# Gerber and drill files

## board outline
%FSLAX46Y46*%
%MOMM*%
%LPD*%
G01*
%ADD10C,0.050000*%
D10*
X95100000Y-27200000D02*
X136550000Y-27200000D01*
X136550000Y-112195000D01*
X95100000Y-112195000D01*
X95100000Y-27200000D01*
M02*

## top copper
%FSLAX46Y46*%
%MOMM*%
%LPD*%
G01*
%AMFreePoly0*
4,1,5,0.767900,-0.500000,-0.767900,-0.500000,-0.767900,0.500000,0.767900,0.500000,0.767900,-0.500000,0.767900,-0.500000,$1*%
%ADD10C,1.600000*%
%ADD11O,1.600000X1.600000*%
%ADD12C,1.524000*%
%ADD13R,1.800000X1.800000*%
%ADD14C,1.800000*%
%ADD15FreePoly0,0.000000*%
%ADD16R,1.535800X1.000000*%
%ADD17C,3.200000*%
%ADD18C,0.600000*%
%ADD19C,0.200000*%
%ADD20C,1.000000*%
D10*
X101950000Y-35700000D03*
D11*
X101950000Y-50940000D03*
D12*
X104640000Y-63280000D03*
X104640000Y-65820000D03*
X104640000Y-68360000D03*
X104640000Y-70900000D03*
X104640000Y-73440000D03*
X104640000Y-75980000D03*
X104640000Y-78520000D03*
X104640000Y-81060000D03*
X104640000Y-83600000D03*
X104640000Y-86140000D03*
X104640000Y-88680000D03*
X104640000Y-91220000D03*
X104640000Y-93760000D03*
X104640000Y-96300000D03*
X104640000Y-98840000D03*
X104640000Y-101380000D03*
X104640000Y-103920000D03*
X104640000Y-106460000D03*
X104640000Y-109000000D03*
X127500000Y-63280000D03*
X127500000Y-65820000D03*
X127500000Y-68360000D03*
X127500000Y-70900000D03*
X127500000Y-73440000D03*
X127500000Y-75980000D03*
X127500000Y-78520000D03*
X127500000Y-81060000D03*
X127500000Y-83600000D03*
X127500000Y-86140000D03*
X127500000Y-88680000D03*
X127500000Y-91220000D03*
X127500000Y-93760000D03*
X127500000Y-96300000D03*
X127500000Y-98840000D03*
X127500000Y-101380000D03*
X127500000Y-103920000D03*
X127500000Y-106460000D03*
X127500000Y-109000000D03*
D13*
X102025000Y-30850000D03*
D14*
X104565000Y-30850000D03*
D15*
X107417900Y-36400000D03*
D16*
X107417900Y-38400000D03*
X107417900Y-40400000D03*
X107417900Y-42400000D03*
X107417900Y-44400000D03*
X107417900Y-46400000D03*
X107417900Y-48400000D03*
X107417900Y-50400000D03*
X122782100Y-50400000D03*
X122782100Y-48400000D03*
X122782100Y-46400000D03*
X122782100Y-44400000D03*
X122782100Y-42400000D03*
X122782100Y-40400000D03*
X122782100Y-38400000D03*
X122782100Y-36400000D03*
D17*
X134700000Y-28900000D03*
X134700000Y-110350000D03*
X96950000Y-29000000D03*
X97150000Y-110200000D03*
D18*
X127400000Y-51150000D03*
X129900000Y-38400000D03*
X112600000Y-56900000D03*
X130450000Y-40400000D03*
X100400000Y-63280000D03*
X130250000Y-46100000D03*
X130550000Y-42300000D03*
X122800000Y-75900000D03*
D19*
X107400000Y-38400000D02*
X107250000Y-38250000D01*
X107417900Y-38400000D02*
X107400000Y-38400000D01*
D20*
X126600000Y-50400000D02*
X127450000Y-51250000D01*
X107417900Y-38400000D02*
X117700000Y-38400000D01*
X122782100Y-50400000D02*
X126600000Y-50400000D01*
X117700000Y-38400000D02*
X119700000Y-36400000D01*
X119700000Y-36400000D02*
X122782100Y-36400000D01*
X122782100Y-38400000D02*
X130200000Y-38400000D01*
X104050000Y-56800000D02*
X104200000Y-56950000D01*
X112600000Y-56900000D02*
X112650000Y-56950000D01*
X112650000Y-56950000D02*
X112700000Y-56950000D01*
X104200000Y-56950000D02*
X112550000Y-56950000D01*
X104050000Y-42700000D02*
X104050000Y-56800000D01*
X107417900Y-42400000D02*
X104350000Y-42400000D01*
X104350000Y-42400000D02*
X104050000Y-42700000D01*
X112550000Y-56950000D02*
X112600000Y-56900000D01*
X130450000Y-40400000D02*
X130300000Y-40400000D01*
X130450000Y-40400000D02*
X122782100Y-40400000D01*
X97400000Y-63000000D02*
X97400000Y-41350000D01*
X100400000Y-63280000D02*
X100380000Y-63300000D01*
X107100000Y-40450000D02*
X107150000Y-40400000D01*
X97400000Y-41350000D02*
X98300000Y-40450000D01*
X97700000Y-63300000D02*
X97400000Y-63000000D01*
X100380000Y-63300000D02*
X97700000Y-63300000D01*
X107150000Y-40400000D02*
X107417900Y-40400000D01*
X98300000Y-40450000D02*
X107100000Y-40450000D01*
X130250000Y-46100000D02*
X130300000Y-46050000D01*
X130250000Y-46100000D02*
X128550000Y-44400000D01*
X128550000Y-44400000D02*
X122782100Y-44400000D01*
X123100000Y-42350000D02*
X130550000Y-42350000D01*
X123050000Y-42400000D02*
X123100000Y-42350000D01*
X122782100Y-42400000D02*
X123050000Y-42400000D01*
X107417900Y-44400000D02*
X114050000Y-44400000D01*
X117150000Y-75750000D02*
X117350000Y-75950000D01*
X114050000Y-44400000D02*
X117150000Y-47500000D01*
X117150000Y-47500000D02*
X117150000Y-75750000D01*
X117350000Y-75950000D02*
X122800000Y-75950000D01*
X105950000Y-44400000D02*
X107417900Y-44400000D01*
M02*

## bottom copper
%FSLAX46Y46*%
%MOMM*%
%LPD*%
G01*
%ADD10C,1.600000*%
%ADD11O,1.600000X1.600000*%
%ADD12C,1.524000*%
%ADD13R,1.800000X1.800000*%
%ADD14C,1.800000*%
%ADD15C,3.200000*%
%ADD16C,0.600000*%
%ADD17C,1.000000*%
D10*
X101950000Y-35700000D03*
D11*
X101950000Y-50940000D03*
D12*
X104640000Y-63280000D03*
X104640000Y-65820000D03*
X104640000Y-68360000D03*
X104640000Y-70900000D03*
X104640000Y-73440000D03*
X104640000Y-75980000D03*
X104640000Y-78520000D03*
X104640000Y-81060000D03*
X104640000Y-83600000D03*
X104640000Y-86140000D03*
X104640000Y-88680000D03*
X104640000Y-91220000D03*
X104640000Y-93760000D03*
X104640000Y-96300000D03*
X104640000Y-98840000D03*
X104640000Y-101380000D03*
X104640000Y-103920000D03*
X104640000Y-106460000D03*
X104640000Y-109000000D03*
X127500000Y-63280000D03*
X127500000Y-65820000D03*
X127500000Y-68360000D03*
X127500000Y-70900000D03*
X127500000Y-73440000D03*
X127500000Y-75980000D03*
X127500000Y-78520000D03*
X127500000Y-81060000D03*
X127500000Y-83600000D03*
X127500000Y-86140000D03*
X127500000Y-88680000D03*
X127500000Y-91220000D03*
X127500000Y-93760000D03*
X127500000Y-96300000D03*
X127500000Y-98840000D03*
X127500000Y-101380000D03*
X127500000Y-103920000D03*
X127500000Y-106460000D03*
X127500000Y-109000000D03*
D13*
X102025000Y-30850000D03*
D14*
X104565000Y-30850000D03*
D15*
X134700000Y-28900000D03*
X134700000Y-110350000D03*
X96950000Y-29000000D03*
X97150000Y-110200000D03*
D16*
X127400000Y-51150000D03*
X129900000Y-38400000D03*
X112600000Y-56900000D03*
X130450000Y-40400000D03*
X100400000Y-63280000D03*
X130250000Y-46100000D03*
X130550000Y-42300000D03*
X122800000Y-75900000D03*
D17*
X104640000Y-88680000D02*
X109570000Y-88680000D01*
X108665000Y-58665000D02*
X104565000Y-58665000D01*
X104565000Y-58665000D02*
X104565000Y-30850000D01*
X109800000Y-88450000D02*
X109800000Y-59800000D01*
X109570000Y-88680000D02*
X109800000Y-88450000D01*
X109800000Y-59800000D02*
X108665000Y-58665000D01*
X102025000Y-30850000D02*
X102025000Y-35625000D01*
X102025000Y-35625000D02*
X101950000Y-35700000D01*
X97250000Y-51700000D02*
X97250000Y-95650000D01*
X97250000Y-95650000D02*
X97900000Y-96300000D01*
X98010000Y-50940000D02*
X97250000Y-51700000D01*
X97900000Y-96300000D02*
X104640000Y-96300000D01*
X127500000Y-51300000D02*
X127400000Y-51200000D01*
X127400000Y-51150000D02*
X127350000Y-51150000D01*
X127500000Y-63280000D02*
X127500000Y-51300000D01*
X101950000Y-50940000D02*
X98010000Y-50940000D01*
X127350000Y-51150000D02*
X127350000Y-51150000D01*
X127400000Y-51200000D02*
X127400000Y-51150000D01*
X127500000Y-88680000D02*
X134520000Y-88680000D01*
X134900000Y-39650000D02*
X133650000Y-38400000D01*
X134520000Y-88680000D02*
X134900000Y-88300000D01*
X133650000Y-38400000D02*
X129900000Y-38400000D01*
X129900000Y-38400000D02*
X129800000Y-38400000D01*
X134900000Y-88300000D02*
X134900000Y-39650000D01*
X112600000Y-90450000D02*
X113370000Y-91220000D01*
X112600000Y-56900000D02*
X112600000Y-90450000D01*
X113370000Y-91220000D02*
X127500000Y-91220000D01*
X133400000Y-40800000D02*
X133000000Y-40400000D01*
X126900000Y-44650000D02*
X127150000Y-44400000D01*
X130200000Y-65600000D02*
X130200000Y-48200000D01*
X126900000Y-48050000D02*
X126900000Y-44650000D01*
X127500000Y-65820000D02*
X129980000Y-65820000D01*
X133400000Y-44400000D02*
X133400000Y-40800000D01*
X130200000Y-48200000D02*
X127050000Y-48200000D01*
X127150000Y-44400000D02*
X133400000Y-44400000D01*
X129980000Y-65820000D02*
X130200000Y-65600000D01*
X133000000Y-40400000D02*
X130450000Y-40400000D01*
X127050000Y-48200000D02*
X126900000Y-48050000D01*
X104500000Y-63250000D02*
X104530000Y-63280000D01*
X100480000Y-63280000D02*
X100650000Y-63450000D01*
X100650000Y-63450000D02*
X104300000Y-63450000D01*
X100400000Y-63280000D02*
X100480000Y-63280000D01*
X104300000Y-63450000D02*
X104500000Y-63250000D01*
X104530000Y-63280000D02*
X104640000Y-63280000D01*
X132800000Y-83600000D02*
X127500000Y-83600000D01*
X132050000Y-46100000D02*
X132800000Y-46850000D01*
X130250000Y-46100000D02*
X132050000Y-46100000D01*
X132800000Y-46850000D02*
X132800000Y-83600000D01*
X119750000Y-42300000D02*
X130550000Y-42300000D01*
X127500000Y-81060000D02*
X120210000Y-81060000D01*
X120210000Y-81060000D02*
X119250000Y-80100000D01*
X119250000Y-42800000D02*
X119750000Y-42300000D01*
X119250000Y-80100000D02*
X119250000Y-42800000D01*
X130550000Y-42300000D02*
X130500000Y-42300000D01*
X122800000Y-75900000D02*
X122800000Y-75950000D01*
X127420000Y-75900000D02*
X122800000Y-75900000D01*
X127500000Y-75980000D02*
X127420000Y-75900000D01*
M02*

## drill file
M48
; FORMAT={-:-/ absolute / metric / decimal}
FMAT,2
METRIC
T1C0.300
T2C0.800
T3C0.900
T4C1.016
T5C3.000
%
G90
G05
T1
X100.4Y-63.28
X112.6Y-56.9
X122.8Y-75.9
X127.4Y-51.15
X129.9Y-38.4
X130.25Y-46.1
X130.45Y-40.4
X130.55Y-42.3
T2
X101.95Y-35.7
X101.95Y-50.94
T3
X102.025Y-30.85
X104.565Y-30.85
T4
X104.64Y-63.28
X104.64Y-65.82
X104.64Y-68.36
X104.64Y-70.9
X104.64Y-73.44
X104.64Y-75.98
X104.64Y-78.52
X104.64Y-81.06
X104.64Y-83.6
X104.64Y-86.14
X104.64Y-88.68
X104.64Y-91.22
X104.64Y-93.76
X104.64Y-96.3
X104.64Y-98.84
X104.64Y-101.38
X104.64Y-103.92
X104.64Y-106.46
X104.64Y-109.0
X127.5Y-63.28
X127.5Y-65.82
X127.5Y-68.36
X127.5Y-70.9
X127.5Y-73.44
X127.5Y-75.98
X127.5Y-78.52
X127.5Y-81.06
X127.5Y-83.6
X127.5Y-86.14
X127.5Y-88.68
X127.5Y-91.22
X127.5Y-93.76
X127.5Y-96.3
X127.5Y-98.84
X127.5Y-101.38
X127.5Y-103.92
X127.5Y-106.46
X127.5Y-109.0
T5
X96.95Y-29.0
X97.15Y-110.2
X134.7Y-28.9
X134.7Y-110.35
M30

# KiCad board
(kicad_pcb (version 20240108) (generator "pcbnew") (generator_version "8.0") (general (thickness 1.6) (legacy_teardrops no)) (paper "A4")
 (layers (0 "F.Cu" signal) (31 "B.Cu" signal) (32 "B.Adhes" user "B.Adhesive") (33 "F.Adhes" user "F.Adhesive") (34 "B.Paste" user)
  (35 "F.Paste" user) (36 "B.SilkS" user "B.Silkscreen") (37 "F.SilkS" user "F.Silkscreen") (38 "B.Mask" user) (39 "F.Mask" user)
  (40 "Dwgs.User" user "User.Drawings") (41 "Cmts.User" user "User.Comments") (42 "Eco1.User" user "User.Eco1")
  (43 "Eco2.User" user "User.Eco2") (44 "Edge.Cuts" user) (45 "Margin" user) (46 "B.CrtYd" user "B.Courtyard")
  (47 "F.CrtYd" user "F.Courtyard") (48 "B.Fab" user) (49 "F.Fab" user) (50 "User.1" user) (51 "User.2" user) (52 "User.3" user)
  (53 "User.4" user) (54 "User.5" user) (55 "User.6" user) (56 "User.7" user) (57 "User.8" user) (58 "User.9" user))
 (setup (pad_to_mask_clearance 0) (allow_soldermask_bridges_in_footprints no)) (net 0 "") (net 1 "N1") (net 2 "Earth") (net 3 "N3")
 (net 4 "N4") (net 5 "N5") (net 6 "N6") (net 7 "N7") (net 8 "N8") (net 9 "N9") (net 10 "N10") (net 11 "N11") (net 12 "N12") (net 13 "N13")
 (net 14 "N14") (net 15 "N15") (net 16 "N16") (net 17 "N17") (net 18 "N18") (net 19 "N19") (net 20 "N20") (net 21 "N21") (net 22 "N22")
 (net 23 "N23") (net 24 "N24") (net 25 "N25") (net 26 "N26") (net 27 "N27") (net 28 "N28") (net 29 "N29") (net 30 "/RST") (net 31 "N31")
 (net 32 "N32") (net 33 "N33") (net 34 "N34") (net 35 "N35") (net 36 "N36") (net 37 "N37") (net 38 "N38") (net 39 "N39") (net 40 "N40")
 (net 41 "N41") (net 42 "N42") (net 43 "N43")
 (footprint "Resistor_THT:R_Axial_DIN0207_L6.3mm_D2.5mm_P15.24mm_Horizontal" (layer "F.Cu") (at 101.95 35.7 -90)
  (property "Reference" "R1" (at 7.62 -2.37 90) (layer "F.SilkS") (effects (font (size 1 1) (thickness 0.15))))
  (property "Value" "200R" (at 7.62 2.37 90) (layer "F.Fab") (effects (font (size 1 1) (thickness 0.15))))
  (pad "1" thru_hole circle (at 0 0 270) (size 1.6 1.6) (drill 0.8) (layers "*.Cu" "*.Mask") (remove_unused_layers no) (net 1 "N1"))
  (pad "2" thru_hole oval (at 15.24 0 270) (size 1.6 1.6) (drill 0.8) (layers "*.Cu" "*.Mask") (remove_unused_layers no) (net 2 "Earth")))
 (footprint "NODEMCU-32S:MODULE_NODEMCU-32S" (layer "F.Cu") (at 116.07 86.14)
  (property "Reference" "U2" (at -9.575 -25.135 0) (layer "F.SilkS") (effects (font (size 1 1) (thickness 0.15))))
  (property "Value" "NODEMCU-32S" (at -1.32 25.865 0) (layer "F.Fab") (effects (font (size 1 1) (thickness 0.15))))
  (pad "J1_1" thru_hole circle (at -11.43 -22.86) (size 1.524 1.524) (drill 1.016) (layers "*.Cu" "*.Mask") (remove_unused_layers no)
   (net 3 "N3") (solder_mask_margin 0.102))
  (pad "J1_2" thru_hole circle (at -11.43 -20.32) (size 1.524 1.524) (drill 1.016) (layers "*.Cu" "*.Mask") (remove_unused_layers no)
   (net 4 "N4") (solder_mask_margin 0.102))
  (pad "J1_3" thru_hole circle (at -11.43 -17.78) (size 1.524 1.524) (drill 1.016) (layers "*.Cu" "*.Mask") (remove_unused_layers no)
   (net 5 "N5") (solder_mask_margin 0.102))
  (pad "J1_4" thru_hole circle (at -11.43 -15.24) (size 1.524 1.524) (drill 1.016) (layers "*.Cu" "*.Mask") (remove_unused_layers no)
   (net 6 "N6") (solder_mask_margin 0.102))
  (pad "J1_5" thru_hole circle (at -11.43 -12.7) (size 1.524 1.524) (drill 1.016) (layers "*.Cu" "*.Mask") (remove_unused_layers no)
   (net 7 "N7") (solder_mask_margin 0.102))
  (pad "J1_6" thru_hole circle (at -11.43 -10.16) (size 1.524 1.524) (drill 1.016) (layers "*.Cu" "*.Mask") (remove_unused_layers no)
   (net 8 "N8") (solder_mask_margin 0.102))
  (pad "J1_7" thru_hole circle (at -11.43 -7.62) (size 1.524 1.524) (drill 1.016) (layers "*.Cu" "*.Mask") (remove_unused_layers no)
   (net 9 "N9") (solder_mask_margin 0.102))
  (pad "J1_8" thru_hole circle (at -11.43 -5.08) (size 1.524 1.524) (drill 1.016) (layers "*.Cu" "*.Mask") (remove_unused_layers no)
   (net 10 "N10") (solder_mask_margin 0.102))
  (pad "J1_9" thru_hole circle (at -11.43 -2.54) (size 1.524 1.524) (drill 1.016) (layers "*.Cu" "*.Mask") (remove_unused_layers no)
   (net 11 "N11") (solder_mask_margin 0.102))
  (pad "J1_10" thru_hole circle (at -11.43 0) (size 1.524 1.524) (drill 1.016) (layers "*.Cu" "*.Mask") (remove_unused_layers no)
   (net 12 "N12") (solder_mask_margin 0.102))
  (pad "J1_11" thru_hole circle (at -11.43 2.54) (size 1.524 1.524) (drill 1.016) (layers "*.Cu" "*.Mask") (remove_unused_layers no)
   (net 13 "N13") (solder_mask_margin 0.102))
  (pad "J1_12" thru_hole circle (at -11.43 5.08) (size 1.524 1.524) (drill 1.016) (layers "*.Cu" "*.Mask") (remove_unused_layers no)
   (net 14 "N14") (solder_mask_margin 0.102))
  (pad "J1_13" thru_hole circle (at -11.43 7.62) (size 1.524 1.524) (drill 1.016) (layers "*.Cu" "*.Mask") (remove_unused_layers no)
   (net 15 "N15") (solder_mask_margin 0.102))
  (pad "J1_14" thru_hole circle (at -11.43 10.16) (size 1.524 1.524) (drill 1.016) (layers "*.Cu" "*.Mask") (remove_unused_layers no)
   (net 2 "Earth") (solder_mask_margin 0.102))
  (pad "J1_15" thru_hole circle (at -11.43 12.7) (size 1.524 1.524) (drill 1.016) (layers "*.Cu" "*.Mask") (remove_unused_layers no)
   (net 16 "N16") (solder_mask_margin 0.102))
  (pad "J1_16" thru_hole circle (at -11.43 15.24) (size 1.524 1.524) (drill 1.016) (layers "*.Cu" "*.Mask") (remove_unused_layers no)
   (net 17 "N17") (solder_mask_margin 0.102))
  (pad "J1_17" thru_hole circle (at -11.43 17.78) (size 1.524 1.524) (drill 1.016) (layers "*.Cu" "*.Mask") (remove_unused_layers no)
   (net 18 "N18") (solder_mask_margin 0.102))
  (pad "J1_18" thru_hole circle (at -11.43 20.32) (size 1.524 1.524) (drill 1.016) (layers "*.Cu" "*.Mask") (remove_unused_layers no)
   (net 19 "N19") (solder_mask_margin 0.102))
  (pad "J1_19" thru_hole circle (at -11.43 22.86) (size 1.524 1.524) (drill 1.016) (layers "*.Cu" "*.Mask") (remove_unused_layers no)
   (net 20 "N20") (solder_mask_margin 0.102))
  (pad "J2_1" thru_hole circle (at 11.43 -22.86) (size 1.524 1.524) (drill 1.016) (layers "*.Cu" "*.Mask") (remove_unused_layers no)
   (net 2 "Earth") (solder_mask_margin 0.102))
  (pad "J2_2" thru_hole circle (at 11.43 -20.32) (size 1.524 1.524) (drill 1.016) (layers "*.Cu" "*.Mask") (remove_unused_layers no)
   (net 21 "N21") (solder_mask_margin 0.102))
  (pad "J2_3" thru_hole circle (at 11.43 -17.78) (size 1.524 1.524) (drill 1.016) (layers "*.Cu" "*.Mask") (remove_unused_layers no)
   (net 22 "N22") (solder_mask_margin 0.102))
  (pad "J2_4" thru_hole circle (at 11.43 -15.24) (size 1.524 1.524) (drill 1.016) (layers "*.Cu" "*.Mask") (remove_unused_layers no)
   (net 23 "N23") (solder_mask_margin 0.102))
  (pad "J2_5" thru_hole circle (at 11.43 -12.7) (size 1.524 1.524) (drill 1.016) (layers "*.Cu" "*.Mask") (remove_unused_layers no)
   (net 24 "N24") (solder_mask_margin 0.102))
  (pad "J2_6" thru_hole circle (at 11.43 -10.16) (size 1.524 1.524) (drill 1.016) (layers "*.Cu" "*.Mask") (remove_unused_layers no)
   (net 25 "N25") (solder_mask_margin 0.102))
  (pad "J2_7" thru_hole circle (at 11.43 -7.62) (size 1.524 1.524) (drill 1.016) (layers "*.Cu" "*.Mask") (remove_unused_layers no)
   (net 2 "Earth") (solder_mask_margin 0.102))
  (pad "J2_8" thru_hole circle (at 11.43 -5.08) (size 1.524 1.524) (drill 1.016) (layers "*.Cu" "*.Mask") (remove_unused_layers no)
   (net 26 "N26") (solder_mask_margin 0.102))
  (pad "J2_9" thru_hole circle (at 11.43 -2.54) (size 1.524 1.524) (drill 1.016) (layers "*.Cu" "*.Mask") (remove_unused_layers no)
   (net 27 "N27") (solder_mask_margin 0.102))
  (pad "J2_10" thru_hole circle (at 11.43 0) (size 1.524 1.524) (drill 1.016) (layers "*.Cu" "*.Mask") (remove_unused_layers no)
   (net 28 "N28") (solder_mask_margin 0.102))
  (pad "J2_11" thru_hole circle (at 11.43 2.54) (size 1.524 1.524) (drill 1.016) (layers "*.Cu" "*.Mask") (remove_unused_layers no)
   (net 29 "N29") (solder_mask_margin 0.102))
  (pad "J2_12" thru_hole circle (at 11.43 5.08) (size 1.524 1.524) (drill 1.016) (layers "*.Cu" "*.Mask") (remove_unused_layers no)
   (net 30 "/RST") (solder_mask_margin 0.102))
  (pad "J2_13" thru_hole circle (at 11.43 7.62) (size 1.524 1.524) (drill 1.016) (layers "*.Cu" "*.Mask") (remove_unused_layers no)
   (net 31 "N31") (solder_mask_margin 0.102))
  (pad "J2_14" thru_hole circle (at 11.43 10.16) (size 1.524 1.524) (drill 1.016) (layers "*.Cu" "*.Mask") (remove_unused_layers no)
   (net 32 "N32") (solder_mask_margin 0.102))
  (pad "J2_15" thru_hole circle (at 11.43 12.7) (size 1.524 1.524) (drill 1.016) (layers "*.Cu" "*.Mask") (remove_unused_layers no)
   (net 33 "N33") (solder_mask_margin 0.102))
  (pad "J2_16" thru_hole circle (at 11.43 15.24) (size 1.524 1.524) (drill 1.016) (layers "*.Cu" "*.Mask") (remove_unused_layers no)
   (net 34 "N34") (solder_mask_margin 0.102))
  (pad "J2_17" thru_hole circle (at 11.43 17.78) (size 1.524 1.524) (drill 1.016) (layers "*.Cu" "*.Mask") (remove_unused_layers no)
   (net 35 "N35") (solder_mask_margin 0.102))
  (pad "J2_18" thru_hole circle (at 11.43 20.32) (size 1.524 1.524) (drill 1.016) (layers "*.Cu" "*.Mask") (remove_unused_layers no)
   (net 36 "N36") (solder_mask_margin 0.102))
  (pad "J2_19" thru_hole circle (at 11.43 22.86) (size 1.524 1.524) (drill 1.016) (layers "*.Cu" "*.Mask") (remove_unused_layers no)
   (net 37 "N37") (solder_mask_margin 0.102)))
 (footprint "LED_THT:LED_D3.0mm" (layer "F.Cu") (at 102.025 30.85)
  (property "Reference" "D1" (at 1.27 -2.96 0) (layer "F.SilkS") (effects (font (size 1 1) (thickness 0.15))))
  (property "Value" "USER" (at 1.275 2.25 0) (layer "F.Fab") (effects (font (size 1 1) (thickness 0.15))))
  (pad "1" thru_hole rect (at 0 0) (size 1.8 1.8) (drill 0.9) (layers "*.Cu" "*.Mask") (remove_unused_layers no) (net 1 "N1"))
  (pad "2" thru_hole circle (at 2.54 0) (size 1.8 1.8) (drill 0.9) (layers "*.Cu" "*.Mask") (remove_unused_layers no) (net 13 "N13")))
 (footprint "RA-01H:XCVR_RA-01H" (layer "F.Cu") (at 115.1 43.4)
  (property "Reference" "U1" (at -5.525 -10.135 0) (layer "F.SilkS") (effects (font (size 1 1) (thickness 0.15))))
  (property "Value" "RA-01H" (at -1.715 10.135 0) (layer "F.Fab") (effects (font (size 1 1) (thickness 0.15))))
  (pad "1" smd custom (at -7.6821 -7) (size 1.5358 1) (layers "F.Cu") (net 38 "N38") (options (clearance outline) (anchor rect))
   (primitives))
  (pad "2" smd rect (at -7.6821 -5) (size 1.5358 1) (layers "F.Cu" "F.Paste" "F.Mask") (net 2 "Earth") (solder_mask_margin 0.102))
  (pad "3" smd rect (at -7.6821 -3) (size 1.5358 1) (layers "F.Cu" "F.Paste" "F.Mask") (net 3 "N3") (solder_mask_margin 0.102))
  (pad "4" smd rect (at -7.6821 -1) (size 1.5358 1) (layers "F.Cu" "F.Paste" "F.Mask") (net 30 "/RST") (solder_mask_margin 0.102))
  (pad "5" smd rect (at -7.6821 1) (size 1.5358 1) (layers "F.Cu" "F.Paste" "F.Mask") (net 25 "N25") (solder_mask_margin 0.102))
  (pad "6" smd rect (at -7.6821 3) (size 1.5358 1) (layers "F.Cu" "F.Paste" "F.Mask") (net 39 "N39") (solder_mask_margin 0.102))
  (pad "7" smd rect (at -7.6821 5) (size 1.5358 1) (layers "F.Cu" "F.Paste" "F.Mask") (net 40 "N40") (solder_mask_margin 0.102))
  (pad "8" smd rect (at -7.6821 7) (size 1.5358 1) (layers "F.Cu" "F.Paste" "F.Mask") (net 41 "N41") (solder_mask_margin 0.102))
  (pad "9" smd rect (at 7.6821 7) (size 1.5358 1) (layers "F.Cu" "F.Paste" "F.Mask") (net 2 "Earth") (solder_mask_margin 0.102))
  (pad "10" smd rect (at 7.6821 5) (size 1.5358 1) (layers "F.Cu" "F.Paste" "F.Mask") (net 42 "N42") (solder_mask_margin 0.102))
  (pad "11" smd rect (at 7.6821 3) (size 1.5358 1) (layers "F.Cu" "F.Paste" "F.Mask") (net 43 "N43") (solder_mask_margin 0.102))
  (pad "12" smd rect (at 7.6821 1) (size 1.5358 1) (layers "F.Cu" "F.Paste" "F.Mask") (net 27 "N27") (solder_mask_margin 0.102))
  (pad "13" smd rect (at 7.6821 -1) (size 1.5358 1) (layers "F.Cu" "F.Paste" "F.Mask") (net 26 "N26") (solder_mask_margin 0.102))
  (pad "14" smd rect (at 7.6821 -3) (size 1.5358 1) (layers "F.Cu" "F.Paste" "F.Mask") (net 21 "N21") (solder_mask_margin 0.102))
  (pad "15" smd rect (at 7.6821 -5) (size 1.5358 1) (layers "F.Cu" "F.Paste" "F.Mask") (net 29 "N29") (solder_mask_margin 0.102))
  (pad "16" smd rect (at 7.6821 -7) (size 1.5358 1) (layers "F.Cu" "F.Paste" "F.Mask") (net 2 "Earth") (solder_mask_margin 0.102)))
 (gr_rect (start 95.1 27.2) (end 136.55 112.195) (stroke (width 0.05) (type default)) (fill none) (layer "Edge.Cuts"))
 (via (at 134.7 28.9) (size 3.2) (drill 3) (layers "F.Cu" "B.Cu") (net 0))
 (via (at 134.7 110.35) (size 3.2) (drill 3) (layers "F.Cu" "B.Cu") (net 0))
 (via (at 96.95 29) (size 3.2) (drill 3) (layers "F.Cu" "B.Cu") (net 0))
 (via (at 97.15 110.2) (size 3.2) (drill 3) (layers "F.Cu" "B.Cu") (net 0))
 (segment (start 104.64 88.68) (end 109.57 88.68) (width 1) (layer "B.Cu") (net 13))
 (segment (start 108.665 58.665) (end 104.565 58.665) (width 1) (layer "B.Cu") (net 13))
 (segment (start 104.565 58.665) (end 104.565 30.85) (width 1) (layer "B.Cu") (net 13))
 (segment (start 109.8 88.45) (end 109.8 59.8) (width 1) (layer "B.Cu") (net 13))
 (segment (start 109.57 88.68) (end 109.8 88.45) (width 1) (layer "B.Cu") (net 13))
 (segment (start 109.8 59.8) (end 108.665 58.665) (width 1) (layer "B.Cu") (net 13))
 (segment (start 102.025 30.85) (end 102.025 35.625) (width 1) (layer "B.Cu") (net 1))
 (segment (start 102.025 35.625) (end 101.95 35.7) (width 1) (layer "B.Cu") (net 1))
 (segment (start 107.4 38.4) (end 107.25 38.25) (width 0.2) (layer "F.Cu") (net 2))
 (segment (start 107.4179 38.4) (end 107.4 38.4) (width 0.2) (layer "F.Cu") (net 2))
 (segment (start 126.6 50.4) (end 127.45 51.25) (width 1) (layer "F.Cu") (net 2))
 (segment (start 107.4179 38.4) (end 117.7 38.4) (width 1) (layer "F.Cu") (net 2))
 (segment (start 122.7821 50.4) (end 126.6 50.4) (width 1) (layer "F.Cu") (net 2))
 (segment (start 117.7 38.4) (end 119.7 36.4) (width 1) (layer "F.Cu") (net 2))
 (segment (start 119.7 36.4) (end 122.7821 36.4) (width 1) (layer "F.Cu") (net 2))
 (via (at 127.4 51.15) (size 0.6) (drill 0.3) (layers "F.Cu" "B.Cu") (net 2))
 (segment (start 97.25 51.7) (end 97.25 95.65) (width 1) (layer "B.Cu") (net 2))
 (segment (start 97.25 95.65) (end 97.9 96.3) (width 1) (layer "B.Cu") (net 2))
 (segment (start 98.01 50.94) (end 97.25 51.7) (width 1) (layer "B.Cu") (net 2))
 (segment (start 97.9 96.3) (end 104.64 96.3) (width 1) (layer "B.Cu") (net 2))
 (segment (start 127.5 51.3) (end 127.4 51.2) (width 1) (layer "B.Cu") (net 2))
 (segment (start 127.4 51.15) (end 127.35 51.15) (width 1) (layer "B.Cu") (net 2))
 (segment (start 127.5 63.28) (end 127.5 51.3) (width 1) (layer "B.Cu") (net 2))
 (segment (start 101.95 50.94) (end 98.01 50.94) (width 1) (layer "B.Cu") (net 2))
 (segment (start 127.35 51.15) (end 127.35 51.15) (width 1) (layer "B.Cu") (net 2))
 (segment (start 127.4 51.2) (end 127.4 51.15) (width 1) (layer "B.Cu") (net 2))
 (segment (start 122.7821 38.4) (end 130.2 38.4) (width 1) (layer "F.Cu") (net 29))
 (via (at 129.9 38.4) (size 0.6) (drill 0.3) (layers "F.Cu" "B.Cu") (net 29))
 (segment (start 127.5 88.68) (end 134.52 88.68) (width 1) (layer "B.Cu") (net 29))
 (segment (start 134.9 39.65) (end 133.65 38.4) (width 1) (layer "B.Cu") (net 29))
 (segment (start 134.52 88.68) (end 134.9 88.3) (width 1) (layer "B.Cu") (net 29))
 (segment (start 133.65 38.4) (end 129.9 38.4) (width 1) (layer "B.Cu") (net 29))
 (segment (start 129.9 38.4) (end 129.8 38.4) (width 1) (layer "B.Cu") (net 29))
 (segment (start 134.9 88.3) (end 134.9 39.65) (width 1) (layer "B.Cu") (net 29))
 (segment (start 104.05 56.8) (end 104.2 56.95) (width 1) (layer "F.Cu") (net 30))
 (segment (start 112.6 56.9) (end 112.65 56.95) (width 1) (layer "F.Cu") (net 30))
 (segment (start 112.65 56.95) (end 112.7 56.95) (width 1) (layer "F.Cu") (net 30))
 (segment (start 104.2 56.95) (end 112.55 56.95) (width 1) (layer "F.Cu") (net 30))
 (segment (start 104.05 42.7) (end 104.05 56.8) (width 1) (layer "F.Cu") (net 30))
 (segment (start 107.4179 42.4) (end 104.35 42.4) (width 1) (layer "F.Cu") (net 30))
 (segment (start 104.35 42.4) (end 104.05 42.7) (width 1) (layer "F.Cu") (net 30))
 (segment (start 112.55 56.95) (end 112.6 56.9) (width 1) (layer "F.Cu") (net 30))
 (via (at 112.6 56.9) (size 0.6) (drill 0.3) (layers "F.Cu" "B.Cu") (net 30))
 (segment (start 112.6 90.45) (end 113.37 91.22) (width 1) (layer "B.Cu") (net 30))
 (segment (start 112.6 56.9) (end 112.6 90.45) (width 1) (layer "B.Cu") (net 30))
 (segment (start 113.37 91.22) (end 127.5 91.22) (width 1) (layer "B.Cu") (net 30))
 (segment (start 130.45 40.4) (end 130.3 40.4) (width 1) (layer "F.Cu") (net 21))
 (segment (start 130.45 40.4) (end 122.7821 40.4) (width 1) (layer "F.Cu") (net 21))
 (via (at 130.45 40.4) (size 0.6) (drill 0.3) (layers "F.Cu" "B.Cu") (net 21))
 (segment (start 133.4 40.8) (end 133 40.4) (width 1) (layer "B.Cu") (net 21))
 (segment (start 126.9 44.65) (end 127.15 44.4) (width 1) (layer "B.Cu") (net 21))
 (segment (start 130.2 65.6) (end 130.2 48.2) (width 1) (layer "B.Cu") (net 21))
 (segment (start 126.9 48.05) (end 126.9 44.65) (width 1) (layer "B.Cu") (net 21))
 (segment (start 127.5 65.82) (end 129.98 65.82) (width 1) (layer "B.Cu") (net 21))
 (segment (start 133.4 44.4) (end 133.4 40.8) (width 1) (layer "B.Cu") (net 21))
 (segment (start 130.2 48.2) (end 127.05 48.2) (width 1) (layer "B.Cu") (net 21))
 (segment (start 127.15 44.4) (end 133.4 44.4) (width 1) (layer "B.Cu") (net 21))
 (segment (start 129.98 65.82) (end 130.2 65.6) (width 1) (layer "B.Cu") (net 21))
 (segment (start 133 40.4) (end 130.45 40.4) (width 1) (layer "B.Cu") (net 21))
 (segment (start 127.05 48.2) (end 126.9 48.05) (width 1) (layer "B.Cu") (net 21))
 (segment (start 97.4 63) (end 97.4 41.35) (width 1) (layer "F.Cu") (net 3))
 (segment (start 100.4 63.28) (end 100.38 63.3) (width 1) (layer "F.Cu") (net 3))
 (segment (start 107.1 40.45) (end 107.15 40.4) (width 1) (layer "F.Cu") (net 3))
 (segment (start 97.4 41.35) (end 98.3 40.45) (width 1) (layer "F.Cu") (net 3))
 (segment (start 97.7 63.3) (end 97.4 63) (width 1) (layer "F.Cu") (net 3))
 (segment (start 100.38 63.3) (end 97.7 63.3) (width 1) (layer "F.Cu") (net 3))
 (segment (start 107.15 40.4) (end 107.4179 40.4) (width 1) (layer "F.Cu") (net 3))
 (segment (start 98.3 40.45) (end 107.1 40.45) (width 1) (layer "F.Cu") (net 3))
 (via (at 100.4 63.28) (size 0.6) (drill 0.3) (layers "F.Cu" "B.Cu") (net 3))
 (segment (start 104.5 63.25) (end 104.53 63.28) (width 1) (layer "B.Cu") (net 3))
 (segment (start 100.48 63.28) (end 100.65 63.45) (width 1) (layer "B.Cu") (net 3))
 (segment (start 100.65 63.45) (end 104.3 63.45) (width 1) (layer "B.Cu") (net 3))
 (segment (start 100.4 63.28) (end 100.48 63.28) (width 1) (layer "B.Cu") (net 3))
 (segment (start 104.3 63.45) (end 104.5 63.25) (width 1) (layer "B.Cu") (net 3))
 (segment (start 104.53 63.28) (end 104.64 63.28) (width 1) (layer "B.Cu") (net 3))
 (segment (start 130.25 46.1) (end 130.3 46.05) (width 1) (layer "F.Cu") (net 27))
 (segment (start 130.25 46.1) (end 128.55 44.4) (width 1) (layer "F.Cu") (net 27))
 (segment (start 128.55 44.4) (end 122.7821 44.4) (width 1) (layer "F.Cu") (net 27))
 (via (at 130.25 46.1) (size 0.6) (drill 0.3) (layers "F.Cu" "B.Cu") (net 27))
 (segment (start 132.8 83.6) (end 127.5 83.6) (width 1) (layer "B.Cu") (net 27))
 (segment (start 132.05 46.1) (end 132.8 46.85) (width 1) (layer "B.Cu") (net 27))
 (segment (start 130.25 46.1) (end 132.05 46.1) (width 1) (layer "B.Cu") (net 27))
 (segment (start 132.8 46.85) (end 132.8 83.6) (width 1) (layer "B.Cu") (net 27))
 (segment (start 123.1 42.35) (end 130.55 42.35) (width 1) (layer "F.Cu") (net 26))
 (segment (start 123.05 42.4) (end 123.1 42.35) (width 1) (layer "F.Cu") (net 26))
 (segment (start 122.7821 42.4) (end 123.05 42.4) (width 1) (layer "F.Cu") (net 26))
 (via (at 130.55 42.3) (size 0.6) (drill 0.3) (layers "F.Cu" "B.Cu") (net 26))
 (segment (start 119.75 42.3) (end 130.55 42.3) (width 1) (layer "B.Cu") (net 26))
 (segment (start 127.5 81.06) (end 120.21 81.06) (width 1) (layer "B.Cu") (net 26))
 (segment (start 120.21 81.06) (end 119.25 80.1) (width 1) (layer "B.Cu") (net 26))
 (segment (start 119.25 42.8) (end 119.75 42.3) (width 1) (layer "B.Cu") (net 26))
 (segment (start 119.25 80.1) (end 119.25 42.8) (width 1) (layer "B.Cu") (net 26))
 (segment (start 130.55 42.3) (end 130.5 42.3) (width 1) (layer "B.Cu") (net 26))
 (segment (start 107.4179 44.4) (end 114.05 44.4) (width 1) (layer "F.Cu") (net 25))
 (segment (start 117.15 75.75) (end 117.35 75.95) (width 1) (layer "F.Cu") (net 25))
 (segment (start 114.05 44.4) (end 117.15 47.5) (width 1) (layer "F.Cu") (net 25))
 (segment (start 117.15 47.5) (end 117.15 75.75) (width 1) (layer "F.Cu") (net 25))
 (segment (start 117.35 75.95) (end 122.8 75.95) (width 1) (layer "F.Cu") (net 25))
 (segment (start 105.95 44.4) (end 107.4179 44.4) (width 1) (layer "F.Cu") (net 25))
 (via (at 122.8 75.9) (size 0.6) (drill 0.3) (layers "F.Cu" "B.Cu") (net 25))
 (segment (start 122.8 75.9) (end 122.8 75.95) (width 1) (layer "B.Cu") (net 25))
 (segment (start 127.42 75.9) (end 122.8 75.9) (width 1) (layer "B.Cu") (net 25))
 (segment (start 127.5 75.98) (end 127.42 75.9) (width 1) (layer "B.Cu") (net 25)))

